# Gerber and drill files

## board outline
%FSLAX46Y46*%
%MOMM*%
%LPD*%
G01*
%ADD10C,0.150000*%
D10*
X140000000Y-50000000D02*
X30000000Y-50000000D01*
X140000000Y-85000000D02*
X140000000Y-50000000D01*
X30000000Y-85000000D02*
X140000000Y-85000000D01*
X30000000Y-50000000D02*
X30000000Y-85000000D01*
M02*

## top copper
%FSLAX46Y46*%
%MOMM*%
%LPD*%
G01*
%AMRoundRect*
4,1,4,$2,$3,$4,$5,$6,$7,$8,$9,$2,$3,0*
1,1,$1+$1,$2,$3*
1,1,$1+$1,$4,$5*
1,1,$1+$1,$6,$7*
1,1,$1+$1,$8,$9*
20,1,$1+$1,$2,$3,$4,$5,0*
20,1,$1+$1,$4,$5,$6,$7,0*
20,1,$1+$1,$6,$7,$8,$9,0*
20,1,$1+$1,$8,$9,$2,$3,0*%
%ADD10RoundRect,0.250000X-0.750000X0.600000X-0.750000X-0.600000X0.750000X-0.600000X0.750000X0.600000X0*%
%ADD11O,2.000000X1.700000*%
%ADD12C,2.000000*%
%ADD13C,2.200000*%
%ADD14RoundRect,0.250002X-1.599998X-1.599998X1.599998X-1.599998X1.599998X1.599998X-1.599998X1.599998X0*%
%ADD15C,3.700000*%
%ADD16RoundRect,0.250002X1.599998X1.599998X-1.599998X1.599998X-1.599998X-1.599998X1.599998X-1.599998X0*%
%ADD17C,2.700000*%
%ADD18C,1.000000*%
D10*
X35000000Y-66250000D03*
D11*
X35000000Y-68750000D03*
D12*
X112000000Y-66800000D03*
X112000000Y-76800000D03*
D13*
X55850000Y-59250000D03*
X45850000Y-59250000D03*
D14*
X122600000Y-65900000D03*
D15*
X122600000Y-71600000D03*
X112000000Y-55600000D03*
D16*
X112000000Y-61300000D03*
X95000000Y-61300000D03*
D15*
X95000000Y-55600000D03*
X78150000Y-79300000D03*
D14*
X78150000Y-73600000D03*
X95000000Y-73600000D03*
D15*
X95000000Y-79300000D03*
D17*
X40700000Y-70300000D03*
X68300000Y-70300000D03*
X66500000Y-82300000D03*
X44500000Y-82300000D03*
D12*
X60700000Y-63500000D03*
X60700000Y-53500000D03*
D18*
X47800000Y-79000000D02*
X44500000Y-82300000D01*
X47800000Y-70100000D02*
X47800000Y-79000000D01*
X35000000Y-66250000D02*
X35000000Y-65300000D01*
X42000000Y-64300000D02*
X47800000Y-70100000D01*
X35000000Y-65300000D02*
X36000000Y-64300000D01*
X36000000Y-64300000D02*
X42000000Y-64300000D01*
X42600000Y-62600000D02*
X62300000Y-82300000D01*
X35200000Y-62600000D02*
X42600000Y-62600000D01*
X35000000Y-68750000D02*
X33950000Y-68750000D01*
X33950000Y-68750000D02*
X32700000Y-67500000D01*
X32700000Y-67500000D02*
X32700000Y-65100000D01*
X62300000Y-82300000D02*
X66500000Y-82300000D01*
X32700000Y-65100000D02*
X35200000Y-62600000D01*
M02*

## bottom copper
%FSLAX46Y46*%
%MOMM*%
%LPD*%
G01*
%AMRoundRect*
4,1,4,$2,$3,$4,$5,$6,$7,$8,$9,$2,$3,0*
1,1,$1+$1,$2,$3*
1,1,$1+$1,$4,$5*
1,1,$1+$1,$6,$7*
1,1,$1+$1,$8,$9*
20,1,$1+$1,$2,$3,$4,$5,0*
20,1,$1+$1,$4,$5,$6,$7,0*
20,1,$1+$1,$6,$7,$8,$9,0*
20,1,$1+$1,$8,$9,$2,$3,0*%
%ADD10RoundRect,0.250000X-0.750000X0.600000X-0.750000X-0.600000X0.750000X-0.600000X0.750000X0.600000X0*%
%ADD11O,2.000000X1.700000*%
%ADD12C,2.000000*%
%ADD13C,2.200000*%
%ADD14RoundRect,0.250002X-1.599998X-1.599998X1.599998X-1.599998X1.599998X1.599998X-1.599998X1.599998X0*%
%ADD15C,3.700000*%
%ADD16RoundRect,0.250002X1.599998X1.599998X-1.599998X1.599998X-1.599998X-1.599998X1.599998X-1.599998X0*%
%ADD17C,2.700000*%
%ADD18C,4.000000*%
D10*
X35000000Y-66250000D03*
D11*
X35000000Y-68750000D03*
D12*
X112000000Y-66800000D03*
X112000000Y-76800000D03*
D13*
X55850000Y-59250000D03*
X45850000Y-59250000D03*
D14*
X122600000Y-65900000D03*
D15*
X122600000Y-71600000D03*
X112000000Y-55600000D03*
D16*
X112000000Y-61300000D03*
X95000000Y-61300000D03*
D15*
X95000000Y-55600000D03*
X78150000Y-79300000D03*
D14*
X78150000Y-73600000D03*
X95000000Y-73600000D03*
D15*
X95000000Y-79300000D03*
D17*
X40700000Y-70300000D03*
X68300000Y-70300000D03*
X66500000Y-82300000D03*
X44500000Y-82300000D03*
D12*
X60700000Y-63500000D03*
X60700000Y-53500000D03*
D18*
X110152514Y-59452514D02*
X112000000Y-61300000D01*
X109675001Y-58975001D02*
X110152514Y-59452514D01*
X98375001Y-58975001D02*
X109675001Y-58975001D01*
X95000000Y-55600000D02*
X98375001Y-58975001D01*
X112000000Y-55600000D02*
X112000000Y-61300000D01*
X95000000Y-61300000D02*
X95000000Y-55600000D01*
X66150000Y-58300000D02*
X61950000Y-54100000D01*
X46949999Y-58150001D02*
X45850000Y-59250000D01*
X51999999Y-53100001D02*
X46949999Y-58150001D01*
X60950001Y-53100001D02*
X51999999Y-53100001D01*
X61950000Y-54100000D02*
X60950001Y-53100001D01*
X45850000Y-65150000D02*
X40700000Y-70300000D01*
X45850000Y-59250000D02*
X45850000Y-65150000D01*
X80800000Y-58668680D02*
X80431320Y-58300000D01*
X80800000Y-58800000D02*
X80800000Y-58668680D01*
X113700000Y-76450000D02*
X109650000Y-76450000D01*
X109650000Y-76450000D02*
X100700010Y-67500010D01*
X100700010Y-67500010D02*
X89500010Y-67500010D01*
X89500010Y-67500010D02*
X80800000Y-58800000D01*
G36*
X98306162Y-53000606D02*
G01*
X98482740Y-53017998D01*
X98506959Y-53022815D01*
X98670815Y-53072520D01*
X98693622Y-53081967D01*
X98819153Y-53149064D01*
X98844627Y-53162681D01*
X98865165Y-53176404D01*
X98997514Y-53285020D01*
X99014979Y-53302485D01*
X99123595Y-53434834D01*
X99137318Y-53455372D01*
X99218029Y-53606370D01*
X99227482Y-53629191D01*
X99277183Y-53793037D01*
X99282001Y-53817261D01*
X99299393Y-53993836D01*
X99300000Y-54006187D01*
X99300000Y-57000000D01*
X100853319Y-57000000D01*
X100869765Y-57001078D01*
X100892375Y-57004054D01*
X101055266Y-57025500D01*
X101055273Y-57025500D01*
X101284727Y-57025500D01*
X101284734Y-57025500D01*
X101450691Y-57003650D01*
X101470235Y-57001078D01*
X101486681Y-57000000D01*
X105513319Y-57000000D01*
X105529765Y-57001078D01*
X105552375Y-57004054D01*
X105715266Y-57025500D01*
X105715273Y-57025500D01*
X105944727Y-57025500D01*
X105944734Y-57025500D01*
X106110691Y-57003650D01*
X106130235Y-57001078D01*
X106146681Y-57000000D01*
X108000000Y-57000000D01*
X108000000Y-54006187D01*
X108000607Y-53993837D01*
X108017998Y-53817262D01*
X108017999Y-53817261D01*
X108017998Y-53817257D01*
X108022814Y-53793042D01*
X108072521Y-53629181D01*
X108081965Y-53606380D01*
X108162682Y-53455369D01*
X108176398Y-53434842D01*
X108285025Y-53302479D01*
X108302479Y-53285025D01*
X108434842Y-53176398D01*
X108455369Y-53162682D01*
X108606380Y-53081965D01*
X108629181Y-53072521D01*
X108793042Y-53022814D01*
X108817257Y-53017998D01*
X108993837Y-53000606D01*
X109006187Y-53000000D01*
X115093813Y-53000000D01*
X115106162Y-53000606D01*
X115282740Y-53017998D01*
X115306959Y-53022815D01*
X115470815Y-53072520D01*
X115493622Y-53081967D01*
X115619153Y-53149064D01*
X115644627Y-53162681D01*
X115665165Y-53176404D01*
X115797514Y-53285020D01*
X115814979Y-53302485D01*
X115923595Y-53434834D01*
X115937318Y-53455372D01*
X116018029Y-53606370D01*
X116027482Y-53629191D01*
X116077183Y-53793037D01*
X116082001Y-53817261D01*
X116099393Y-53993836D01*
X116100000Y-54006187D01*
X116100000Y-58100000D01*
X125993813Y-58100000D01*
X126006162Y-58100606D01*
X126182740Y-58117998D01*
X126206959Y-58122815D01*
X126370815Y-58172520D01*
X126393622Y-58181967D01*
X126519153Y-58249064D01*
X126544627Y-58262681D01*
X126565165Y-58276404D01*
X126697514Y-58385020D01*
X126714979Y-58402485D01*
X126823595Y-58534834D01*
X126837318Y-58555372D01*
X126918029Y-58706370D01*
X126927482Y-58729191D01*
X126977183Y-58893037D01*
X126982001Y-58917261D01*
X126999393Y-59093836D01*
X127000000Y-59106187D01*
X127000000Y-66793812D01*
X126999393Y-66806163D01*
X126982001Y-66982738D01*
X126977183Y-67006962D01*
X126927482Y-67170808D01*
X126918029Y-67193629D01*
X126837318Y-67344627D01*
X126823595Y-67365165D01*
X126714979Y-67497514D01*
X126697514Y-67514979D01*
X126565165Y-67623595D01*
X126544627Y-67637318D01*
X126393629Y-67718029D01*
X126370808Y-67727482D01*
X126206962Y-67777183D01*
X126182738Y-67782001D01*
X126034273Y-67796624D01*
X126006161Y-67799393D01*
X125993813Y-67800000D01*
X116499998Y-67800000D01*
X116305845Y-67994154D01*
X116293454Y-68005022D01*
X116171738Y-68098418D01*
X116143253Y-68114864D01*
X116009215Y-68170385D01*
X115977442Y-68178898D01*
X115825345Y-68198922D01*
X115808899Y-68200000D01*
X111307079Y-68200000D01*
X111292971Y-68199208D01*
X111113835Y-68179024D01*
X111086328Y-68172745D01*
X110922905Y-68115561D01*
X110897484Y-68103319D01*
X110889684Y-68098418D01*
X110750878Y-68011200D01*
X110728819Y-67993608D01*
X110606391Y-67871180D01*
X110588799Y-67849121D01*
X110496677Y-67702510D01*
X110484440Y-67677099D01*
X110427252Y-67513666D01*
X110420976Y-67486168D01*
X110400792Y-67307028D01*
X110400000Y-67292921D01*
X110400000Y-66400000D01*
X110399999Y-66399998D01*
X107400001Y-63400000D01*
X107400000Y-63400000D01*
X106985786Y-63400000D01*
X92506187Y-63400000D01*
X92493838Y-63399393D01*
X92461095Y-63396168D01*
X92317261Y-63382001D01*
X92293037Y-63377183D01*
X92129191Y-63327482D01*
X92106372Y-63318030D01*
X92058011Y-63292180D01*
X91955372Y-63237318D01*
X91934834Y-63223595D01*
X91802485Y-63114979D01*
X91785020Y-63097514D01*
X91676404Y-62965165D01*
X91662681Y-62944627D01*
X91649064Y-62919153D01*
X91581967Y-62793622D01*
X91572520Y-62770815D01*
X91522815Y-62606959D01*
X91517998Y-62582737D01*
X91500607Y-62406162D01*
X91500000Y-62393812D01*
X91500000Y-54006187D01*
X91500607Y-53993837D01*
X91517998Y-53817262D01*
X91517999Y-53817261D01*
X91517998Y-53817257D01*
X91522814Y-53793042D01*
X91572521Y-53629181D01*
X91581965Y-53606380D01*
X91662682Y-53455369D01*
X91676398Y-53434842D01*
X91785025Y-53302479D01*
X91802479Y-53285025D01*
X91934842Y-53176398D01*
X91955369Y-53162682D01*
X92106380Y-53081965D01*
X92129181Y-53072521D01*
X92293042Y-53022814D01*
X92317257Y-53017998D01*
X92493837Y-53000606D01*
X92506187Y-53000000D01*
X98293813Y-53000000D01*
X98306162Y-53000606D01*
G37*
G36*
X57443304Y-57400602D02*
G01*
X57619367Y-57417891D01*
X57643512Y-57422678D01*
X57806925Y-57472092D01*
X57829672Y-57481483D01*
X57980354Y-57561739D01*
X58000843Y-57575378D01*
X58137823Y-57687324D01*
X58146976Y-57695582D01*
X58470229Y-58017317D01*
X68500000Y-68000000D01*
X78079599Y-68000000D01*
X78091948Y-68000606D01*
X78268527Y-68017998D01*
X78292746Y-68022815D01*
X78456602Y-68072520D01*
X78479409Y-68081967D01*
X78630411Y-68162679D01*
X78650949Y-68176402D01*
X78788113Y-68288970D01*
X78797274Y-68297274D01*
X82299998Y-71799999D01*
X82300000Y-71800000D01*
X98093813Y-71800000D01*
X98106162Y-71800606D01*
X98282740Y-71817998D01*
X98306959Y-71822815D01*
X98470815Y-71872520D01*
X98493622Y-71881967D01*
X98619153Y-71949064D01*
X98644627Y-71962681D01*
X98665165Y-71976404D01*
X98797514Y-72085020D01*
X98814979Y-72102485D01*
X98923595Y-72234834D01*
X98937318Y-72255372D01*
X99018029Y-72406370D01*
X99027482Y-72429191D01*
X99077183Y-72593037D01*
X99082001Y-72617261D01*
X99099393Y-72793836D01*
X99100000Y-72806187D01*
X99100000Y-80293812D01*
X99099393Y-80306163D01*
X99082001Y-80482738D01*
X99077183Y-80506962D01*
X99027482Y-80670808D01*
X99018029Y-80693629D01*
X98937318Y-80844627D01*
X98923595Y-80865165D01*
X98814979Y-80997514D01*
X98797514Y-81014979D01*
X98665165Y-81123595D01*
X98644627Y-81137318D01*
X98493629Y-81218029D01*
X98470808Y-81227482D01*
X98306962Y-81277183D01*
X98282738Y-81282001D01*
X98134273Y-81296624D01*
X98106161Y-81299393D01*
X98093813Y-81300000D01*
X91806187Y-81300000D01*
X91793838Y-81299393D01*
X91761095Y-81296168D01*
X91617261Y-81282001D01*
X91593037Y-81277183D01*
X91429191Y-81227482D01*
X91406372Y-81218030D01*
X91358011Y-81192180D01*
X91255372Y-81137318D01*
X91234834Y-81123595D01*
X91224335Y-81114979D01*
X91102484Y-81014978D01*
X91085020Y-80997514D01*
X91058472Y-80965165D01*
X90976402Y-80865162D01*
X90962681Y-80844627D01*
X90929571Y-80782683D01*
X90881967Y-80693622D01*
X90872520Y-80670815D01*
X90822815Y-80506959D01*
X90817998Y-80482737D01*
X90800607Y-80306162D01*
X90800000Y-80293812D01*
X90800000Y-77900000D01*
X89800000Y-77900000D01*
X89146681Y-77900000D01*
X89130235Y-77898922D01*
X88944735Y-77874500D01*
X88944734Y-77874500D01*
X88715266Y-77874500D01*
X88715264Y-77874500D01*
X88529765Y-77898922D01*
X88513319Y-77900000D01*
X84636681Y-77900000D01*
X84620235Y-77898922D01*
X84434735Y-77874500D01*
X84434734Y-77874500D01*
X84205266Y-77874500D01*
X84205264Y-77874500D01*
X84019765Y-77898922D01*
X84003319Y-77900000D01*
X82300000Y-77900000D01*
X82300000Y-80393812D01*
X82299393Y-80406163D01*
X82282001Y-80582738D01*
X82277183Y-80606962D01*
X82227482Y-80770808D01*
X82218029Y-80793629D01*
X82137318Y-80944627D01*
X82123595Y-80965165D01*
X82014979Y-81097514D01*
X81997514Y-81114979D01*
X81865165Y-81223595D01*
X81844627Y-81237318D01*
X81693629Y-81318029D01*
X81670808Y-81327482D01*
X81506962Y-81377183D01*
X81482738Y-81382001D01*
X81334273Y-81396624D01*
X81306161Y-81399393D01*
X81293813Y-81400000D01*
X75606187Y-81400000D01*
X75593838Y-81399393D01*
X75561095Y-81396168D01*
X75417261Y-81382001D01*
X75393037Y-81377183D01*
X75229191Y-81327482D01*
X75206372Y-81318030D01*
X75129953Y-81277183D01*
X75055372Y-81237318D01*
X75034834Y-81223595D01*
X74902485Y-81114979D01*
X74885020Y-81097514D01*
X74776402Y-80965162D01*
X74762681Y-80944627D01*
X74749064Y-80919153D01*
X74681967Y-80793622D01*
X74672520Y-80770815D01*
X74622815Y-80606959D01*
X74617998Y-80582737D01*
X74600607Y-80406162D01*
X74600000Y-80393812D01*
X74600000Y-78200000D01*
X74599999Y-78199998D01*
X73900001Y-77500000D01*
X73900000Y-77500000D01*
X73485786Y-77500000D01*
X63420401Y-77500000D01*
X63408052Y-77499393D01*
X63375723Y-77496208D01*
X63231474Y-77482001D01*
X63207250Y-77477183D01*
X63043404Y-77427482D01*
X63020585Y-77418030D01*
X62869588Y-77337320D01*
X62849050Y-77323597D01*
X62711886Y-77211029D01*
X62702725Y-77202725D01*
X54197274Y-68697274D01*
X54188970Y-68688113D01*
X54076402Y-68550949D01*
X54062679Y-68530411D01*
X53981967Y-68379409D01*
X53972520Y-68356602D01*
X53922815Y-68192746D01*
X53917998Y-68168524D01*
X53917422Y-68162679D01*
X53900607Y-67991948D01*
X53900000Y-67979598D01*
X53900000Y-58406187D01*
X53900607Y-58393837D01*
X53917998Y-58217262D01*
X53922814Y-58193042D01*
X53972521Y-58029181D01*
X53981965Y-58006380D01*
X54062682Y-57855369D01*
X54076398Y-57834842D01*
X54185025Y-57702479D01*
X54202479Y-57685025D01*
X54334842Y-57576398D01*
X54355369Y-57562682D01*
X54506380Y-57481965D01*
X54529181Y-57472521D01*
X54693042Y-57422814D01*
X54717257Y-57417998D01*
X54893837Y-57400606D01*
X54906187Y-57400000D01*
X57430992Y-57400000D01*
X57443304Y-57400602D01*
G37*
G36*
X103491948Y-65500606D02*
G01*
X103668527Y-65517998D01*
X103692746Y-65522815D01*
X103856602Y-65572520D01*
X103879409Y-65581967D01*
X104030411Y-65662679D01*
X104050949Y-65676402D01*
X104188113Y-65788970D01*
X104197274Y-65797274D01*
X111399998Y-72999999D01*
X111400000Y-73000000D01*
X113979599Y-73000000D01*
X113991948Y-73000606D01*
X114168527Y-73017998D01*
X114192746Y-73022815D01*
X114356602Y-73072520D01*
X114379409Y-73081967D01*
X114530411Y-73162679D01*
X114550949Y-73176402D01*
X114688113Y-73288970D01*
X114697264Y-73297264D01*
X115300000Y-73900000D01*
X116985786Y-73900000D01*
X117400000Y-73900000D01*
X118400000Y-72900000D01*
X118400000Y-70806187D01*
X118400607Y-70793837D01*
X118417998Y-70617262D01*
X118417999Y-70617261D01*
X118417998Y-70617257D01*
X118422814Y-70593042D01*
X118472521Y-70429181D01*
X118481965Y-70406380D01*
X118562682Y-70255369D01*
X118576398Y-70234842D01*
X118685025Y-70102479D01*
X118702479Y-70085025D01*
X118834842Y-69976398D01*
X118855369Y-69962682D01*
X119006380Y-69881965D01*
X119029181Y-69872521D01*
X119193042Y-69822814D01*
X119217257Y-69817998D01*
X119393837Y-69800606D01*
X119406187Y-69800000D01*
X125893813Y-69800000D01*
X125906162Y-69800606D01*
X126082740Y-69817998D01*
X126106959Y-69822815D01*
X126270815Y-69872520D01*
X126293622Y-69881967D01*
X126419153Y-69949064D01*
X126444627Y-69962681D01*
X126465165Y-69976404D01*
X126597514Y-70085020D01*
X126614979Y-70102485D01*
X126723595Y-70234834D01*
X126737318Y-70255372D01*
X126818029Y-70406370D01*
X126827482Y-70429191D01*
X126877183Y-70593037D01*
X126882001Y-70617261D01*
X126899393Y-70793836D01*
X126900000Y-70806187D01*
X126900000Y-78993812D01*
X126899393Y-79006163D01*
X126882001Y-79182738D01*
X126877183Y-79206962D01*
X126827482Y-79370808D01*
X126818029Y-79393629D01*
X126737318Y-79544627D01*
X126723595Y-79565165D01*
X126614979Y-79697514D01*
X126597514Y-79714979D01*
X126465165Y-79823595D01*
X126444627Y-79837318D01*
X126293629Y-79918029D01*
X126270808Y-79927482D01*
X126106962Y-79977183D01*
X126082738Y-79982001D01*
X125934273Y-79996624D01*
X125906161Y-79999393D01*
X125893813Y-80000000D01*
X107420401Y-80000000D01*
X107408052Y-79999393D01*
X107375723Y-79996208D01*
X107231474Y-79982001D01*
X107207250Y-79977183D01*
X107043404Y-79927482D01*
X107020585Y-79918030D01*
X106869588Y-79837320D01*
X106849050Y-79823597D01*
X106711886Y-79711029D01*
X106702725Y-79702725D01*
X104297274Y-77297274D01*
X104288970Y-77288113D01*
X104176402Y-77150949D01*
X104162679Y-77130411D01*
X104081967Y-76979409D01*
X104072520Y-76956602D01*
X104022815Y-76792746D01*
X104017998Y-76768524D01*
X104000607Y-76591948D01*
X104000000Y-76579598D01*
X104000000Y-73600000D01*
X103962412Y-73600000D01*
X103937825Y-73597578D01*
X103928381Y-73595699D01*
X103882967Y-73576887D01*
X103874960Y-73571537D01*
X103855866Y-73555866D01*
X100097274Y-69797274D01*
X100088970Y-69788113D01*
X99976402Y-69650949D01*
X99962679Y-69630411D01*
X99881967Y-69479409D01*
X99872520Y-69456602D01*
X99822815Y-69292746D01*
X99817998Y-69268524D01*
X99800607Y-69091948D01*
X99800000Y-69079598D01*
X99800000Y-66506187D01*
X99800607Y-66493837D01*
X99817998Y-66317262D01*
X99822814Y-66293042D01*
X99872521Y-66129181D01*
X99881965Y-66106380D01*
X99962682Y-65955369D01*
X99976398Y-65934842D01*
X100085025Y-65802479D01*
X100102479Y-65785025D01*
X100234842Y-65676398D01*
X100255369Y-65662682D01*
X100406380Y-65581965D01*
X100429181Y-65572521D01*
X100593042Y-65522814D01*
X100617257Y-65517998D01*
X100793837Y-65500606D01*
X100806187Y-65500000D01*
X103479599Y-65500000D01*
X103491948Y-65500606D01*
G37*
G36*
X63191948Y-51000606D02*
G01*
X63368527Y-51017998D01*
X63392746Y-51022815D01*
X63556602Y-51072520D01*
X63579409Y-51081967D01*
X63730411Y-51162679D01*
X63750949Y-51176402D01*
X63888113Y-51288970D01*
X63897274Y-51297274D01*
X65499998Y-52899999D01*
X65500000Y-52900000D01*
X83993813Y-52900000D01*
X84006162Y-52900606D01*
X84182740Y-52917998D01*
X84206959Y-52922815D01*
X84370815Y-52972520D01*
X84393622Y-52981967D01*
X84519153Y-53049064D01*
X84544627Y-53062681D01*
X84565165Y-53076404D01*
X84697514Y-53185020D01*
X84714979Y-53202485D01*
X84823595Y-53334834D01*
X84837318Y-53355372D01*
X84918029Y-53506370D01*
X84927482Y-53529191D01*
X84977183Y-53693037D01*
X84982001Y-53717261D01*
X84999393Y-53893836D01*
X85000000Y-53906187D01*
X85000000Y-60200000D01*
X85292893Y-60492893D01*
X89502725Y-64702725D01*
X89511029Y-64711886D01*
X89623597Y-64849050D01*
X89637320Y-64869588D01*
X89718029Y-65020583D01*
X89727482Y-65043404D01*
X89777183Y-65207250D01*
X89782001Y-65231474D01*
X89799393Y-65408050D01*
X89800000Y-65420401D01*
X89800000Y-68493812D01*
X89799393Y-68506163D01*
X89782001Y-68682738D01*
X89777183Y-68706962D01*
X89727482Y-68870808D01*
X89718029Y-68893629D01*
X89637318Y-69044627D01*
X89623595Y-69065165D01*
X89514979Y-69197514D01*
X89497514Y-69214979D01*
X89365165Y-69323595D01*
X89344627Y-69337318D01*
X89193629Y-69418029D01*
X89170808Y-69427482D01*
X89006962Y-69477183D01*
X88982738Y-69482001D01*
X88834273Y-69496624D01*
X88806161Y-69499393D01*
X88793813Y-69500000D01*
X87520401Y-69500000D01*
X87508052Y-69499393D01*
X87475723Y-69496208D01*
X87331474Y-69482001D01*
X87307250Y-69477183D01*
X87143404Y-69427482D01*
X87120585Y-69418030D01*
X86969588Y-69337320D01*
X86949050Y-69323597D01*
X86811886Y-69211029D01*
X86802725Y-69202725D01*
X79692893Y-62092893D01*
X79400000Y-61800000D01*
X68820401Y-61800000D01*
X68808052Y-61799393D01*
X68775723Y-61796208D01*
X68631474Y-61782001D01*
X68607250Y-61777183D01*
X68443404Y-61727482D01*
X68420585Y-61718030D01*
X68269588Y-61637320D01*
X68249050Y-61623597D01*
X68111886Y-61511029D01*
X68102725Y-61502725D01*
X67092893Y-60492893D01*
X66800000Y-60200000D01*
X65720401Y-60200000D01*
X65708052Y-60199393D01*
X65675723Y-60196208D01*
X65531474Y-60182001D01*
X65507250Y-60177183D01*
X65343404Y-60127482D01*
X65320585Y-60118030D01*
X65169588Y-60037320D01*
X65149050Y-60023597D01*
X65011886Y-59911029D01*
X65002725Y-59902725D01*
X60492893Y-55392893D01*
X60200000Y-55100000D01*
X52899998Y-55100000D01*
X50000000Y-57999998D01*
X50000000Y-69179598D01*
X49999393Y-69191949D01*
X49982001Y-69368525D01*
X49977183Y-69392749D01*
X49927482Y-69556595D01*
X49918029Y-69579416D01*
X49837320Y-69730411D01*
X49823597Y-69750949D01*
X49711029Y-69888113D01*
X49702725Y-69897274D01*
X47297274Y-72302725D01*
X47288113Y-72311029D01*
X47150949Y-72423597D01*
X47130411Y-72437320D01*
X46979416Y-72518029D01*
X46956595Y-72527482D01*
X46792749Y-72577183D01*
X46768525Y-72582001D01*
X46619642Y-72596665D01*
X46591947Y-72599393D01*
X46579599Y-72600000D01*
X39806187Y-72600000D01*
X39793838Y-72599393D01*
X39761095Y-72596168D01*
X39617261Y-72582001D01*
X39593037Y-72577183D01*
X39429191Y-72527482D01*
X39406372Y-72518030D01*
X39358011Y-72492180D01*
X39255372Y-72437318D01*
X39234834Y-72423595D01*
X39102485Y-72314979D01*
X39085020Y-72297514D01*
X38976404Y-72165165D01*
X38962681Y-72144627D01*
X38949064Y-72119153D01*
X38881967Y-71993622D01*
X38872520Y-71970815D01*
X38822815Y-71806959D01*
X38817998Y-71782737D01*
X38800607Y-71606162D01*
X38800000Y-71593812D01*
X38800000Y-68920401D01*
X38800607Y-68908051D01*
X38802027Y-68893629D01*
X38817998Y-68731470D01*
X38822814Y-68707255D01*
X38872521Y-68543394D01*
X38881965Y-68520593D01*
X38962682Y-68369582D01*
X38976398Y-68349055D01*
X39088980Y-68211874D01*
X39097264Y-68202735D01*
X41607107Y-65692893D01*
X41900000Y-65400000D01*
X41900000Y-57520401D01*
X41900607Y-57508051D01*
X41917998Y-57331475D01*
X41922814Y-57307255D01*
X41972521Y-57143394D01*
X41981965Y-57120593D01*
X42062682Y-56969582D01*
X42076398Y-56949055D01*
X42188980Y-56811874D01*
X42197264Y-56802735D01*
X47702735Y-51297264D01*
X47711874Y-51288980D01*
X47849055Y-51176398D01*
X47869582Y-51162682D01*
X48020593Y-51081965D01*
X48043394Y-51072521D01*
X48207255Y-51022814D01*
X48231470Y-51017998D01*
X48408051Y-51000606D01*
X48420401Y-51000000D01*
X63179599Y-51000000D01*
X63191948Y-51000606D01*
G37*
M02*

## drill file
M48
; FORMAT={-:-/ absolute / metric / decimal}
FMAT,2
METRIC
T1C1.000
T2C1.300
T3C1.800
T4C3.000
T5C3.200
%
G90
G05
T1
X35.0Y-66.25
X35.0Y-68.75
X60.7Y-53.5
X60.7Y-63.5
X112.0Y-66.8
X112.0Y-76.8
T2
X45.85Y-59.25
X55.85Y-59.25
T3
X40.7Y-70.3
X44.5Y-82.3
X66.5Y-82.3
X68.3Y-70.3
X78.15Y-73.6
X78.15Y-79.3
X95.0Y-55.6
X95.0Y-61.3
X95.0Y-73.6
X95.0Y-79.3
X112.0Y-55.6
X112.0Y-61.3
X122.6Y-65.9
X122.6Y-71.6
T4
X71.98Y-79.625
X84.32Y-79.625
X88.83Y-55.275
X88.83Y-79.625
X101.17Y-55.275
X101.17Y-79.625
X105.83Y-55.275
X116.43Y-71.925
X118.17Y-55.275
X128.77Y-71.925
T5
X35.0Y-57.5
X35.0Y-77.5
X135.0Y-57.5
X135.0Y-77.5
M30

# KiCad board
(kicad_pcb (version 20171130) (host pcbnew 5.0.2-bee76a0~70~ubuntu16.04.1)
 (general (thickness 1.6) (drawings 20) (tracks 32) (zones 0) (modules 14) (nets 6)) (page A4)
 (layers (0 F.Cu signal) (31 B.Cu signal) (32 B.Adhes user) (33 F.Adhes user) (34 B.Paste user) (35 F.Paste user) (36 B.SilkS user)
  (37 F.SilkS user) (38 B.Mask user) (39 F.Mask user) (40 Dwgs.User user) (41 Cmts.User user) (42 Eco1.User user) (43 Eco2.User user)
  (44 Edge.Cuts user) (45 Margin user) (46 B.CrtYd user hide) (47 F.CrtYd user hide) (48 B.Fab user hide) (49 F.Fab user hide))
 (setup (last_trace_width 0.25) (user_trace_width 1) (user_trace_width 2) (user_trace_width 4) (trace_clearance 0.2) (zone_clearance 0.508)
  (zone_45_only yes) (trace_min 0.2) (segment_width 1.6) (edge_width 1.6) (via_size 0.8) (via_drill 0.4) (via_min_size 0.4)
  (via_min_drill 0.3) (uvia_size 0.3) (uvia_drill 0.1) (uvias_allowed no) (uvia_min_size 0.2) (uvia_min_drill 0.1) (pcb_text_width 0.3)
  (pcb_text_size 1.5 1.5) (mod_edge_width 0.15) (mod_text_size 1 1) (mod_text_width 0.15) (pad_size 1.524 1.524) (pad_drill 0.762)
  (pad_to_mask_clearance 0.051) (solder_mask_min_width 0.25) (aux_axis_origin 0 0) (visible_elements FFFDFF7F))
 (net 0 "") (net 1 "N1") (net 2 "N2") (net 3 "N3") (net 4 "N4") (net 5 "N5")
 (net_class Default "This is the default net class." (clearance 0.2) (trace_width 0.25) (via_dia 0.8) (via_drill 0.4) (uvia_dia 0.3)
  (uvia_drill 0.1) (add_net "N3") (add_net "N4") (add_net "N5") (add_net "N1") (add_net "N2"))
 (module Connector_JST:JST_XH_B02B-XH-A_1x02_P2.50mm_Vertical (layer F.Cu) (at 35 66.25 270)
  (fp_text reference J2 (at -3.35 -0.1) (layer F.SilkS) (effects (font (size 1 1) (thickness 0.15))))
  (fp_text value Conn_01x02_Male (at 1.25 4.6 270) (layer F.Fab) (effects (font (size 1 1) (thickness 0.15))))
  (pad 1 thru_hole roundrect (at 0 0 270) (size 1.7 2) (drill 1) (layers *.Cu *.Mask) (roundrect_rratio 0.147059) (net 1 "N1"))
  (pad 2 thru_hole oval (at 2.5 0 270) (size 1.7 2) (drill 1) (layers *.Cu *.Mask) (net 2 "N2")))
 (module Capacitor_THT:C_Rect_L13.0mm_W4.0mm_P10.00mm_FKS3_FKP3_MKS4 (layer F.Cu) (at 112 66.8 270)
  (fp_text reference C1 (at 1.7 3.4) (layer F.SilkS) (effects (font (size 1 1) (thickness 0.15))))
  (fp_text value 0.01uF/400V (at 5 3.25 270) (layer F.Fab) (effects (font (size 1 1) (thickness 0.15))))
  (pad 1 thru_hole circle (at 0 0 270) (size 2 2) (drill 1) (layers *.Cu *.Mask) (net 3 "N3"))
  (pad 2 thru_hole circle (at 10 0 270) (size 2 2) (drill 1) (layers *.Cu *.Mask) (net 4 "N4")))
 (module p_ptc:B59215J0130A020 (layer F.Cu) (at 50.85 59.25 270)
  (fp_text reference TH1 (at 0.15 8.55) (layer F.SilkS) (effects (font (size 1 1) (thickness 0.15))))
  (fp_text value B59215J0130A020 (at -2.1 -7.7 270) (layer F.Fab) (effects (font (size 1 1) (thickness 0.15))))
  (pad 1 thru_hole circle (at 0 -5 270) (size 2.2 2.2) (drill 1.3) (layers *.Cu *.Mask) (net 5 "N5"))
  (pad 2 thru_hole circle (at 0 5 270) (size 2.2 2.2) (drill 1.3) (layers *.Cu *.Mask) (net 4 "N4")))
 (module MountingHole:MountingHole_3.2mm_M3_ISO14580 (layer F.Cu) (at 35 77.5)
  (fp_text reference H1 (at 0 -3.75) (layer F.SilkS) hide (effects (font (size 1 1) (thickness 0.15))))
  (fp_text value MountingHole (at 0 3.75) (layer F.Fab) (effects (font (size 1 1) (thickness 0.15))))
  (pad 1 np_thru_hole circle (at 0 0) (size 3.2 3.2) (drill 3.2) (layers *.Cu *.Mask)))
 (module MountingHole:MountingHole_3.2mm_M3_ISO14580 (layer F.Cu) (at 135 77.5)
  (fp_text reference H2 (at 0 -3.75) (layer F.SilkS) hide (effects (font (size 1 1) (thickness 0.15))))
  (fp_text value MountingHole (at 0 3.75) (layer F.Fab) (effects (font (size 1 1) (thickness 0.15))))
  (pad 1 np_thru_hole circle (at 0 0) (size 3.2 3.2) (drill 3.2) (layers *.Cu *.Mask)))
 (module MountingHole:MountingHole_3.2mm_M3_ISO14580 (layer F.Cu) (at 35 57.5)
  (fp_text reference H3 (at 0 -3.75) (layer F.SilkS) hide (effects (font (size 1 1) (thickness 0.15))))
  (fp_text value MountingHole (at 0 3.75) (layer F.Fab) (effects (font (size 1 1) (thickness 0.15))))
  (pad 1 np_thru_hole circle (at 0 0) (size 3.2 3.2) (drill 3.2) (layers *.Cu *.Mask)))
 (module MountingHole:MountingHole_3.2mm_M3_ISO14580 (layer F.Cu) (at 135 57.5)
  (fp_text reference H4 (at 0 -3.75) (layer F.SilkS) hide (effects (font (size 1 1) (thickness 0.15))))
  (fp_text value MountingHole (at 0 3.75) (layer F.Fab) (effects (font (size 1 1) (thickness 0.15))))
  (pad 1 np_thru_hole circle (at 0 0) (size 3.2 3.2) (drill 3.2) (layers *.Cu *.Mask)))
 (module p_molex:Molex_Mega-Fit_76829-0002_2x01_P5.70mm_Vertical (layer F.Cu) (at 122.6 65.9)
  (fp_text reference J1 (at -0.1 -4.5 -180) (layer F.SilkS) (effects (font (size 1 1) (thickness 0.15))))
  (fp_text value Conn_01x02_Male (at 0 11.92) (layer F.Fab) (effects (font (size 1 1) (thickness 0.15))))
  (pad 1 thru_hole roundrect (at 0 0) (size 3.7 3.7) (drill 1.8) (layers *.Cu *.Mask) (roundrect_rratio 0.067568) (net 3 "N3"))
  (pad 2 thru_hole circle (at 0 5.7) (size 3.7 3.7) (drill 1.8) (layers *.Cu *.Mask) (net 4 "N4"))
  (pad "" np_thru_hole circle (at -6.17 6.025) (size 3 3) (drill 3) (layers *.Cu *.Mask))
  (pad "" np_thru_hole circle (at 6.17 6.025) (size 3 3) (drill 3) (layers *.Cu *.Mask)))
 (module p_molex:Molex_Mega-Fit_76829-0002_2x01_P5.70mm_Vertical (layer F.Cu) (at 112 61.3 180)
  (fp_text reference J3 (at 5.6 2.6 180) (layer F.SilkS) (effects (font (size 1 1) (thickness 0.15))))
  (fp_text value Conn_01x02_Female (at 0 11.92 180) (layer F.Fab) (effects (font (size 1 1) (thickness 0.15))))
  (pad "" np_thru_hole circle (at 6.17 6.025 180) (size 3 3) (drill 3) (layers *.Cu *.Mask))
  (pad "" np_thru_hole circle (at -6.17 6.025 180) (size 3 3) (drill 3) (layers *.Cu *.Mask))
  (pad 2 thru_hole circle (at 0 5.7 180) (size 3.7 3.7) (drill 1.8) (layers *.Cu *.Mask) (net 3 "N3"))
  (pad 1 thru_hole roundrect (at 0 0 180) (size 3.7 3.7) (drill 1.8) (layers *.Cu *.Mask) (roundrect_rratio 0.067568) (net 3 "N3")))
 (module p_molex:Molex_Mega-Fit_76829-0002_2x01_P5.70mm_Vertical (layer F.Cu) (at 95 61.3 180)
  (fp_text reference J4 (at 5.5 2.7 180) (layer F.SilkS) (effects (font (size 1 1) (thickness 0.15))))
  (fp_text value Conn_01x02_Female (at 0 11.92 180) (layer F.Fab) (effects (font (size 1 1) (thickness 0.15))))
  (pad 1 thru_hole roundrect (at 0 0 180) (size 3.7 3.7) (drill 1.8) (layers *.Cu *.Mask) (roundrect_rratio 0.067568) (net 3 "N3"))
  (pad 2 thru_hole circle (at 0 5.7 180) (size 3.7 3.7) (drill 1.8) (layers *.Cu *.Mask) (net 3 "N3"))
  (pad "" np_thru_hole circle (at -6.17 6.025 180) (size 3 3) (drill 3) (layers *.Cu *.Mask))
  (pad "" np_thru_hole circle (at 6.17 6.025 180) (size 3 3) (drill 3) (layers *.Cu *.Mask)))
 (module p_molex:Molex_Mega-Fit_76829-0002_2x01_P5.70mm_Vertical (layer F.Cu) (at 78.15 73.6)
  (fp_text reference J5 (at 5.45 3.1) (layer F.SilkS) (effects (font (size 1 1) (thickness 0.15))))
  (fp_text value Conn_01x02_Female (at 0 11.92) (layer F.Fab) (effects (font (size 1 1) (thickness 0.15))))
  (pad "" np_thru_hole circle (at 6.17 6.025) (size 3 3) (drill 3) (layers *.Cu *.Mask))
  (pad "" np_thru_hole circle (at -6.17 6.025) (size 3 3) (drill 3) (layers *.Cu *.Mask))
  (pad 2 thru_hole circle (at 0 5.7) (size 3.7 3.7) (drill 1.8) (layers *.Cu *.Mask) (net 5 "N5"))
  (pad 1 thru_hole roundrect (at 0 0) (size 3.7 3.7) (drill 1.8) (layers *.Cu *.Mask) (roundrect_rratio 0.067568) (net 5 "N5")))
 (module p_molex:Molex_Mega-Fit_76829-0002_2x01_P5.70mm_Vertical (layer F.Cu) (at 95 73.6)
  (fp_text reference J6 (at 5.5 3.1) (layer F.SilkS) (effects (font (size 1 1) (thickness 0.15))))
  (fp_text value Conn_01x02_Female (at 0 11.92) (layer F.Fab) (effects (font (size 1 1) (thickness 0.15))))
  (pad 1 thru_hole roundrect (at 0 0) (size 3.7 3.7) (drill 1.8) (layers *.Cu *.Mask) (roundrect_rratio 0.067568) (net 5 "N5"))
  (pad 2 thru_hole circle (at 0 5.7) (size 3.7 3.7) (drill 1.8) (layers *.Cu *.Mask) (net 5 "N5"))
  (pad "" np_thru_hole circle (at -6.17 6.025) (size 3 3) (drill 3) (layers *.Cu *.Mask))
  (pad "" np_thru_hole circle (at 6.17 6.025) (size 3 3) (drill 3) (layers *.Cu *.Mask)))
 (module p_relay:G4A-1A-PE (layer F.Cu) (at 54.5 76.55)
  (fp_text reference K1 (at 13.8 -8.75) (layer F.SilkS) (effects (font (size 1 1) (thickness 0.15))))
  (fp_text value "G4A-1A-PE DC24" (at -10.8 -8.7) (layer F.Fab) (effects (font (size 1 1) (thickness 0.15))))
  (pad 3 thru_hole circle (at -13.8 -6.25) (size 2.7 2.7) (drill 1.8) (layers *.Cu *.Mask) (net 4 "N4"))
  (pad 2 thru_hole circle (at 13.8 -6.25) (size 2.7 2.7) (drill 1.8) (layers *.Cu *.Mask) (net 5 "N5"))
  (pad 5 thru_hole circle (at 12 5.75) (size 2.7 2.7) (drill 1.8) (layers *.Cu *.Mask) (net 2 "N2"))
  (pad 1 thru_hole circle (at -10 5.75) (size 2.7 2.7) (drill 1.8) (layers *.Cu *.Mask) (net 1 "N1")))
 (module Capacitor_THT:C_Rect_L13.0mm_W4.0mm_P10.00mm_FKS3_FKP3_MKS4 (layer F.Cu) (at 60.7 63.5 90)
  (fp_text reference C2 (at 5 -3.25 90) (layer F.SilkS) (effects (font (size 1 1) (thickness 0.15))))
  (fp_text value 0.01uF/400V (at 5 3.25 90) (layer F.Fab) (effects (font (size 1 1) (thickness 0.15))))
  (pad 1 thru_hole circle (at 0 0 90) (size 2 2) (drill 1) (layers *.Cu *.Mask) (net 5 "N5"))
  (pad 2 thru_hole circle (at 10 0 90) (size 2 2) (drill 1) (layers *.Cu *.Mask) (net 4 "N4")))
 (gr_line (start 140 50) (end 30 50) (layer Edge.Cuts) (width 0.15))
 (gr_line (start 140 85) (end 140 50) (layer Edge.Cuts) (width 0.15))
 (gr_line (start 30 85) (end 140 85) (layer Edge.Cuts) (width 0.15))
 (gr_line (start 30 50) (end 30 85) (layer Edge.Cuts) (width 0.15))
 (segment (start 110.152514 59.452514) (end 112 61.3) (width 4) (layer B.Cu) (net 3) (status 20))
 (segment (start 109.675001 58.975001) (end 110.152514 59.452514) (width 4) (layer B.Cu) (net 3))
 (segment (start 98.375001 58.975001) (end 109.675001 58.975001) (width 4) (layer B.Cu) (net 3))
 (segment (start 95 55.6) (end 98.375001 58.975001) (width 4) (layer B.Cu) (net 3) (status 10))
 (segment (start 112 55.6) (end 112 61.3) (width 4) (layer B.Cu) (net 3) (status 30))
 (segment (start 95 61.3) (end 95 55.6) (width 4) (layer B.Cu) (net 3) (status 30))
 (segment (start 66.15 58.3) (end 61.95 54.1) (width 4) (layer B.Cu) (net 4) (status 20))
 (segment (start 46.949999 58.150001) (end 45.85 59.25) (width 4) (layer B.Cu) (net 4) (status 20))
 (segment (start 51.999999 53.100001) (end 46.949999 58.150001) (width 4) (layer B.Cu) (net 4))
 (segment (start 60.950001 53.100001) (end 51.999999 53.100001) (width 4) (layer B.Cu) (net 4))
 (segment (start 61.95 54.1) (end 60.950001 53.100001) (width 4) (layer B.Cu) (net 4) (status 10))
 (segment (start 45.85 65.15) (end 40.7 70.3) (width 4) (layer B.Cu) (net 4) (status 20))
 (segment (start 45.85 59.25) (end 45.85 65.15) (width 4) (layer B.Cu) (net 4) (status 10))
 (segment (start 80.8 58.66868) (end 80.43132 58.3) (width 4) (layer B.Cu) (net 4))
 (segment (start 80.8 58.8) (end 80.8 58.66868) (width 4) (layer B.Cu) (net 4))
 (segment (start 113.7 76.45) (end 109.65 76.45) (width 4) (layer B.Cu) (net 4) (status 10))
 (segment (start 109.65 76.45) (end 100.70001 67.50001) (width 4) (layer B.Cu) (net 4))
 (segment (start 100.70001 67.50001) (end 89.50001 67.50001) (width 4) (layer B.Cu) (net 4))
 (segment (start 89.50001 67.50001) (end 80.8 58.8) (width 4) (layer B.Cu) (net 4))
 (segment (start 47.8 79) (end 44.5 82.3) (width 1) (layer F.Cu) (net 1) (status 20))
 (segment (start 47.8 70.1) (end 47.8 79) (width 1) (layer F.Cu) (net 1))
 (segment (start 35 66.25) (end 35 65.3) (width 1) (layer F.Cu) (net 1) (status 10))
 (segment (start 42 64.3) (end 47.8 70.1) (width 1) (layer F.Cu) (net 1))
 (segment (start 35 65.3) (end 36 64.3) (width 1) (layer F.Cu) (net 1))
 (segment (start 36 64.3) (end 42 64.3) (width 1) (layer F.Cu) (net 1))
 (segment (start 42.6 62.6) (end 62.3 82.3) (width 1) (layer F.Cu) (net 2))
 (segment (start 35.2 62.6) (end 42.6 62.6) (width 1) (layer F.Cu) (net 2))
 (segment (start 35 68.75) (end 33.95 68.75) (width 1) (layer F.Cu) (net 2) (status 10))
 (segment (start 33.95 68.75) (end 32.7 67.5) (width 1) (layer F.Cu) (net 2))
 (segment (start 32.7 67.5) (end 32.7 65.1) (width 1) (layer F.Cu) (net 2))
 (segment (start 62.3 82.3) (end 66.5 82.3) (width 1) (layer F.Cu) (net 2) (status 20))
 (segment (start 32.7 65.1) (end 35.2 62.6) (width 1) (layer F.Cu) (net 2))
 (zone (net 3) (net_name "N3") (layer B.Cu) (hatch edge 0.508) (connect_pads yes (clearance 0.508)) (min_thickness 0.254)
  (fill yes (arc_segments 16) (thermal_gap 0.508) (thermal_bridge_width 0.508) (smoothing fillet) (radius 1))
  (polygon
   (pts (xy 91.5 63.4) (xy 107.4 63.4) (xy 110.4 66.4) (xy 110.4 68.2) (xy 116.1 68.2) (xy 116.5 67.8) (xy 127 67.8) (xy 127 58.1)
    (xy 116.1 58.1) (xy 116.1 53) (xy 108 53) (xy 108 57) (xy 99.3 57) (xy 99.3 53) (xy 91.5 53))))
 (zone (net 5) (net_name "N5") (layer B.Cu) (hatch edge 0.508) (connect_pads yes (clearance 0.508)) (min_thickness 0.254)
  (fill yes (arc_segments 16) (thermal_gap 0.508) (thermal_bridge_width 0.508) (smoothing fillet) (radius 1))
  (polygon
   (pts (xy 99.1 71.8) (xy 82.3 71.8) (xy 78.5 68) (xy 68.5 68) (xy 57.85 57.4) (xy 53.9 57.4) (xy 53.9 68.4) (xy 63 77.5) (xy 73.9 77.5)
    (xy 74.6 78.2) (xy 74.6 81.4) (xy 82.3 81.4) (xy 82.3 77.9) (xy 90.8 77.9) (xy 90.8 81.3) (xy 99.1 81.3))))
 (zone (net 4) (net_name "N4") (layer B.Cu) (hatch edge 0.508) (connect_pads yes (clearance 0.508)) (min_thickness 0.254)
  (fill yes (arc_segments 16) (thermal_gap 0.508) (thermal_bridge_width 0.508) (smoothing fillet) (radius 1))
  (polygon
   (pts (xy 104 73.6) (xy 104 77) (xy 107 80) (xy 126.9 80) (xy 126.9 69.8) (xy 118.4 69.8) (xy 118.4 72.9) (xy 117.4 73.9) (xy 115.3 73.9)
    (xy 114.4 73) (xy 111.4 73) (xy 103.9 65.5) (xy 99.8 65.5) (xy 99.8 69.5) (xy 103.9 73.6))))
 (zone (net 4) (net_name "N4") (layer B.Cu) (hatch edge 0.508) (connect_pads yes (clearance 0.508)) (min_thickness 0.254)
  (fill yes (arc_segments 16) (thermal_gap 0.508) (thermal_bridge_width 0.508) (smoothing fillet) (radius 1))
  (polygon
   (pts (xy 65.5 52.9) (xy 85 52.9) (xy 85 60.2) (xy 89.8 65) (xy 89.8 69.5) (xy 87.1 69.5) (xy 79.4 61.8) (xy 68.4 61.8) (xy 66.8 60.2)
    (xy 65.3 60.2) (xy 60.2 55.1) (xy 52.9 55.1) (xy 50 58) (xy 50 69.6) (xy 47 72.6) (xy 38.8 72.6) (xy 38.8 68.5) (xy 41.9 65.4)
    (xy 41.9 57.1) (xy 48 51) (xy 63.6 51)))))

